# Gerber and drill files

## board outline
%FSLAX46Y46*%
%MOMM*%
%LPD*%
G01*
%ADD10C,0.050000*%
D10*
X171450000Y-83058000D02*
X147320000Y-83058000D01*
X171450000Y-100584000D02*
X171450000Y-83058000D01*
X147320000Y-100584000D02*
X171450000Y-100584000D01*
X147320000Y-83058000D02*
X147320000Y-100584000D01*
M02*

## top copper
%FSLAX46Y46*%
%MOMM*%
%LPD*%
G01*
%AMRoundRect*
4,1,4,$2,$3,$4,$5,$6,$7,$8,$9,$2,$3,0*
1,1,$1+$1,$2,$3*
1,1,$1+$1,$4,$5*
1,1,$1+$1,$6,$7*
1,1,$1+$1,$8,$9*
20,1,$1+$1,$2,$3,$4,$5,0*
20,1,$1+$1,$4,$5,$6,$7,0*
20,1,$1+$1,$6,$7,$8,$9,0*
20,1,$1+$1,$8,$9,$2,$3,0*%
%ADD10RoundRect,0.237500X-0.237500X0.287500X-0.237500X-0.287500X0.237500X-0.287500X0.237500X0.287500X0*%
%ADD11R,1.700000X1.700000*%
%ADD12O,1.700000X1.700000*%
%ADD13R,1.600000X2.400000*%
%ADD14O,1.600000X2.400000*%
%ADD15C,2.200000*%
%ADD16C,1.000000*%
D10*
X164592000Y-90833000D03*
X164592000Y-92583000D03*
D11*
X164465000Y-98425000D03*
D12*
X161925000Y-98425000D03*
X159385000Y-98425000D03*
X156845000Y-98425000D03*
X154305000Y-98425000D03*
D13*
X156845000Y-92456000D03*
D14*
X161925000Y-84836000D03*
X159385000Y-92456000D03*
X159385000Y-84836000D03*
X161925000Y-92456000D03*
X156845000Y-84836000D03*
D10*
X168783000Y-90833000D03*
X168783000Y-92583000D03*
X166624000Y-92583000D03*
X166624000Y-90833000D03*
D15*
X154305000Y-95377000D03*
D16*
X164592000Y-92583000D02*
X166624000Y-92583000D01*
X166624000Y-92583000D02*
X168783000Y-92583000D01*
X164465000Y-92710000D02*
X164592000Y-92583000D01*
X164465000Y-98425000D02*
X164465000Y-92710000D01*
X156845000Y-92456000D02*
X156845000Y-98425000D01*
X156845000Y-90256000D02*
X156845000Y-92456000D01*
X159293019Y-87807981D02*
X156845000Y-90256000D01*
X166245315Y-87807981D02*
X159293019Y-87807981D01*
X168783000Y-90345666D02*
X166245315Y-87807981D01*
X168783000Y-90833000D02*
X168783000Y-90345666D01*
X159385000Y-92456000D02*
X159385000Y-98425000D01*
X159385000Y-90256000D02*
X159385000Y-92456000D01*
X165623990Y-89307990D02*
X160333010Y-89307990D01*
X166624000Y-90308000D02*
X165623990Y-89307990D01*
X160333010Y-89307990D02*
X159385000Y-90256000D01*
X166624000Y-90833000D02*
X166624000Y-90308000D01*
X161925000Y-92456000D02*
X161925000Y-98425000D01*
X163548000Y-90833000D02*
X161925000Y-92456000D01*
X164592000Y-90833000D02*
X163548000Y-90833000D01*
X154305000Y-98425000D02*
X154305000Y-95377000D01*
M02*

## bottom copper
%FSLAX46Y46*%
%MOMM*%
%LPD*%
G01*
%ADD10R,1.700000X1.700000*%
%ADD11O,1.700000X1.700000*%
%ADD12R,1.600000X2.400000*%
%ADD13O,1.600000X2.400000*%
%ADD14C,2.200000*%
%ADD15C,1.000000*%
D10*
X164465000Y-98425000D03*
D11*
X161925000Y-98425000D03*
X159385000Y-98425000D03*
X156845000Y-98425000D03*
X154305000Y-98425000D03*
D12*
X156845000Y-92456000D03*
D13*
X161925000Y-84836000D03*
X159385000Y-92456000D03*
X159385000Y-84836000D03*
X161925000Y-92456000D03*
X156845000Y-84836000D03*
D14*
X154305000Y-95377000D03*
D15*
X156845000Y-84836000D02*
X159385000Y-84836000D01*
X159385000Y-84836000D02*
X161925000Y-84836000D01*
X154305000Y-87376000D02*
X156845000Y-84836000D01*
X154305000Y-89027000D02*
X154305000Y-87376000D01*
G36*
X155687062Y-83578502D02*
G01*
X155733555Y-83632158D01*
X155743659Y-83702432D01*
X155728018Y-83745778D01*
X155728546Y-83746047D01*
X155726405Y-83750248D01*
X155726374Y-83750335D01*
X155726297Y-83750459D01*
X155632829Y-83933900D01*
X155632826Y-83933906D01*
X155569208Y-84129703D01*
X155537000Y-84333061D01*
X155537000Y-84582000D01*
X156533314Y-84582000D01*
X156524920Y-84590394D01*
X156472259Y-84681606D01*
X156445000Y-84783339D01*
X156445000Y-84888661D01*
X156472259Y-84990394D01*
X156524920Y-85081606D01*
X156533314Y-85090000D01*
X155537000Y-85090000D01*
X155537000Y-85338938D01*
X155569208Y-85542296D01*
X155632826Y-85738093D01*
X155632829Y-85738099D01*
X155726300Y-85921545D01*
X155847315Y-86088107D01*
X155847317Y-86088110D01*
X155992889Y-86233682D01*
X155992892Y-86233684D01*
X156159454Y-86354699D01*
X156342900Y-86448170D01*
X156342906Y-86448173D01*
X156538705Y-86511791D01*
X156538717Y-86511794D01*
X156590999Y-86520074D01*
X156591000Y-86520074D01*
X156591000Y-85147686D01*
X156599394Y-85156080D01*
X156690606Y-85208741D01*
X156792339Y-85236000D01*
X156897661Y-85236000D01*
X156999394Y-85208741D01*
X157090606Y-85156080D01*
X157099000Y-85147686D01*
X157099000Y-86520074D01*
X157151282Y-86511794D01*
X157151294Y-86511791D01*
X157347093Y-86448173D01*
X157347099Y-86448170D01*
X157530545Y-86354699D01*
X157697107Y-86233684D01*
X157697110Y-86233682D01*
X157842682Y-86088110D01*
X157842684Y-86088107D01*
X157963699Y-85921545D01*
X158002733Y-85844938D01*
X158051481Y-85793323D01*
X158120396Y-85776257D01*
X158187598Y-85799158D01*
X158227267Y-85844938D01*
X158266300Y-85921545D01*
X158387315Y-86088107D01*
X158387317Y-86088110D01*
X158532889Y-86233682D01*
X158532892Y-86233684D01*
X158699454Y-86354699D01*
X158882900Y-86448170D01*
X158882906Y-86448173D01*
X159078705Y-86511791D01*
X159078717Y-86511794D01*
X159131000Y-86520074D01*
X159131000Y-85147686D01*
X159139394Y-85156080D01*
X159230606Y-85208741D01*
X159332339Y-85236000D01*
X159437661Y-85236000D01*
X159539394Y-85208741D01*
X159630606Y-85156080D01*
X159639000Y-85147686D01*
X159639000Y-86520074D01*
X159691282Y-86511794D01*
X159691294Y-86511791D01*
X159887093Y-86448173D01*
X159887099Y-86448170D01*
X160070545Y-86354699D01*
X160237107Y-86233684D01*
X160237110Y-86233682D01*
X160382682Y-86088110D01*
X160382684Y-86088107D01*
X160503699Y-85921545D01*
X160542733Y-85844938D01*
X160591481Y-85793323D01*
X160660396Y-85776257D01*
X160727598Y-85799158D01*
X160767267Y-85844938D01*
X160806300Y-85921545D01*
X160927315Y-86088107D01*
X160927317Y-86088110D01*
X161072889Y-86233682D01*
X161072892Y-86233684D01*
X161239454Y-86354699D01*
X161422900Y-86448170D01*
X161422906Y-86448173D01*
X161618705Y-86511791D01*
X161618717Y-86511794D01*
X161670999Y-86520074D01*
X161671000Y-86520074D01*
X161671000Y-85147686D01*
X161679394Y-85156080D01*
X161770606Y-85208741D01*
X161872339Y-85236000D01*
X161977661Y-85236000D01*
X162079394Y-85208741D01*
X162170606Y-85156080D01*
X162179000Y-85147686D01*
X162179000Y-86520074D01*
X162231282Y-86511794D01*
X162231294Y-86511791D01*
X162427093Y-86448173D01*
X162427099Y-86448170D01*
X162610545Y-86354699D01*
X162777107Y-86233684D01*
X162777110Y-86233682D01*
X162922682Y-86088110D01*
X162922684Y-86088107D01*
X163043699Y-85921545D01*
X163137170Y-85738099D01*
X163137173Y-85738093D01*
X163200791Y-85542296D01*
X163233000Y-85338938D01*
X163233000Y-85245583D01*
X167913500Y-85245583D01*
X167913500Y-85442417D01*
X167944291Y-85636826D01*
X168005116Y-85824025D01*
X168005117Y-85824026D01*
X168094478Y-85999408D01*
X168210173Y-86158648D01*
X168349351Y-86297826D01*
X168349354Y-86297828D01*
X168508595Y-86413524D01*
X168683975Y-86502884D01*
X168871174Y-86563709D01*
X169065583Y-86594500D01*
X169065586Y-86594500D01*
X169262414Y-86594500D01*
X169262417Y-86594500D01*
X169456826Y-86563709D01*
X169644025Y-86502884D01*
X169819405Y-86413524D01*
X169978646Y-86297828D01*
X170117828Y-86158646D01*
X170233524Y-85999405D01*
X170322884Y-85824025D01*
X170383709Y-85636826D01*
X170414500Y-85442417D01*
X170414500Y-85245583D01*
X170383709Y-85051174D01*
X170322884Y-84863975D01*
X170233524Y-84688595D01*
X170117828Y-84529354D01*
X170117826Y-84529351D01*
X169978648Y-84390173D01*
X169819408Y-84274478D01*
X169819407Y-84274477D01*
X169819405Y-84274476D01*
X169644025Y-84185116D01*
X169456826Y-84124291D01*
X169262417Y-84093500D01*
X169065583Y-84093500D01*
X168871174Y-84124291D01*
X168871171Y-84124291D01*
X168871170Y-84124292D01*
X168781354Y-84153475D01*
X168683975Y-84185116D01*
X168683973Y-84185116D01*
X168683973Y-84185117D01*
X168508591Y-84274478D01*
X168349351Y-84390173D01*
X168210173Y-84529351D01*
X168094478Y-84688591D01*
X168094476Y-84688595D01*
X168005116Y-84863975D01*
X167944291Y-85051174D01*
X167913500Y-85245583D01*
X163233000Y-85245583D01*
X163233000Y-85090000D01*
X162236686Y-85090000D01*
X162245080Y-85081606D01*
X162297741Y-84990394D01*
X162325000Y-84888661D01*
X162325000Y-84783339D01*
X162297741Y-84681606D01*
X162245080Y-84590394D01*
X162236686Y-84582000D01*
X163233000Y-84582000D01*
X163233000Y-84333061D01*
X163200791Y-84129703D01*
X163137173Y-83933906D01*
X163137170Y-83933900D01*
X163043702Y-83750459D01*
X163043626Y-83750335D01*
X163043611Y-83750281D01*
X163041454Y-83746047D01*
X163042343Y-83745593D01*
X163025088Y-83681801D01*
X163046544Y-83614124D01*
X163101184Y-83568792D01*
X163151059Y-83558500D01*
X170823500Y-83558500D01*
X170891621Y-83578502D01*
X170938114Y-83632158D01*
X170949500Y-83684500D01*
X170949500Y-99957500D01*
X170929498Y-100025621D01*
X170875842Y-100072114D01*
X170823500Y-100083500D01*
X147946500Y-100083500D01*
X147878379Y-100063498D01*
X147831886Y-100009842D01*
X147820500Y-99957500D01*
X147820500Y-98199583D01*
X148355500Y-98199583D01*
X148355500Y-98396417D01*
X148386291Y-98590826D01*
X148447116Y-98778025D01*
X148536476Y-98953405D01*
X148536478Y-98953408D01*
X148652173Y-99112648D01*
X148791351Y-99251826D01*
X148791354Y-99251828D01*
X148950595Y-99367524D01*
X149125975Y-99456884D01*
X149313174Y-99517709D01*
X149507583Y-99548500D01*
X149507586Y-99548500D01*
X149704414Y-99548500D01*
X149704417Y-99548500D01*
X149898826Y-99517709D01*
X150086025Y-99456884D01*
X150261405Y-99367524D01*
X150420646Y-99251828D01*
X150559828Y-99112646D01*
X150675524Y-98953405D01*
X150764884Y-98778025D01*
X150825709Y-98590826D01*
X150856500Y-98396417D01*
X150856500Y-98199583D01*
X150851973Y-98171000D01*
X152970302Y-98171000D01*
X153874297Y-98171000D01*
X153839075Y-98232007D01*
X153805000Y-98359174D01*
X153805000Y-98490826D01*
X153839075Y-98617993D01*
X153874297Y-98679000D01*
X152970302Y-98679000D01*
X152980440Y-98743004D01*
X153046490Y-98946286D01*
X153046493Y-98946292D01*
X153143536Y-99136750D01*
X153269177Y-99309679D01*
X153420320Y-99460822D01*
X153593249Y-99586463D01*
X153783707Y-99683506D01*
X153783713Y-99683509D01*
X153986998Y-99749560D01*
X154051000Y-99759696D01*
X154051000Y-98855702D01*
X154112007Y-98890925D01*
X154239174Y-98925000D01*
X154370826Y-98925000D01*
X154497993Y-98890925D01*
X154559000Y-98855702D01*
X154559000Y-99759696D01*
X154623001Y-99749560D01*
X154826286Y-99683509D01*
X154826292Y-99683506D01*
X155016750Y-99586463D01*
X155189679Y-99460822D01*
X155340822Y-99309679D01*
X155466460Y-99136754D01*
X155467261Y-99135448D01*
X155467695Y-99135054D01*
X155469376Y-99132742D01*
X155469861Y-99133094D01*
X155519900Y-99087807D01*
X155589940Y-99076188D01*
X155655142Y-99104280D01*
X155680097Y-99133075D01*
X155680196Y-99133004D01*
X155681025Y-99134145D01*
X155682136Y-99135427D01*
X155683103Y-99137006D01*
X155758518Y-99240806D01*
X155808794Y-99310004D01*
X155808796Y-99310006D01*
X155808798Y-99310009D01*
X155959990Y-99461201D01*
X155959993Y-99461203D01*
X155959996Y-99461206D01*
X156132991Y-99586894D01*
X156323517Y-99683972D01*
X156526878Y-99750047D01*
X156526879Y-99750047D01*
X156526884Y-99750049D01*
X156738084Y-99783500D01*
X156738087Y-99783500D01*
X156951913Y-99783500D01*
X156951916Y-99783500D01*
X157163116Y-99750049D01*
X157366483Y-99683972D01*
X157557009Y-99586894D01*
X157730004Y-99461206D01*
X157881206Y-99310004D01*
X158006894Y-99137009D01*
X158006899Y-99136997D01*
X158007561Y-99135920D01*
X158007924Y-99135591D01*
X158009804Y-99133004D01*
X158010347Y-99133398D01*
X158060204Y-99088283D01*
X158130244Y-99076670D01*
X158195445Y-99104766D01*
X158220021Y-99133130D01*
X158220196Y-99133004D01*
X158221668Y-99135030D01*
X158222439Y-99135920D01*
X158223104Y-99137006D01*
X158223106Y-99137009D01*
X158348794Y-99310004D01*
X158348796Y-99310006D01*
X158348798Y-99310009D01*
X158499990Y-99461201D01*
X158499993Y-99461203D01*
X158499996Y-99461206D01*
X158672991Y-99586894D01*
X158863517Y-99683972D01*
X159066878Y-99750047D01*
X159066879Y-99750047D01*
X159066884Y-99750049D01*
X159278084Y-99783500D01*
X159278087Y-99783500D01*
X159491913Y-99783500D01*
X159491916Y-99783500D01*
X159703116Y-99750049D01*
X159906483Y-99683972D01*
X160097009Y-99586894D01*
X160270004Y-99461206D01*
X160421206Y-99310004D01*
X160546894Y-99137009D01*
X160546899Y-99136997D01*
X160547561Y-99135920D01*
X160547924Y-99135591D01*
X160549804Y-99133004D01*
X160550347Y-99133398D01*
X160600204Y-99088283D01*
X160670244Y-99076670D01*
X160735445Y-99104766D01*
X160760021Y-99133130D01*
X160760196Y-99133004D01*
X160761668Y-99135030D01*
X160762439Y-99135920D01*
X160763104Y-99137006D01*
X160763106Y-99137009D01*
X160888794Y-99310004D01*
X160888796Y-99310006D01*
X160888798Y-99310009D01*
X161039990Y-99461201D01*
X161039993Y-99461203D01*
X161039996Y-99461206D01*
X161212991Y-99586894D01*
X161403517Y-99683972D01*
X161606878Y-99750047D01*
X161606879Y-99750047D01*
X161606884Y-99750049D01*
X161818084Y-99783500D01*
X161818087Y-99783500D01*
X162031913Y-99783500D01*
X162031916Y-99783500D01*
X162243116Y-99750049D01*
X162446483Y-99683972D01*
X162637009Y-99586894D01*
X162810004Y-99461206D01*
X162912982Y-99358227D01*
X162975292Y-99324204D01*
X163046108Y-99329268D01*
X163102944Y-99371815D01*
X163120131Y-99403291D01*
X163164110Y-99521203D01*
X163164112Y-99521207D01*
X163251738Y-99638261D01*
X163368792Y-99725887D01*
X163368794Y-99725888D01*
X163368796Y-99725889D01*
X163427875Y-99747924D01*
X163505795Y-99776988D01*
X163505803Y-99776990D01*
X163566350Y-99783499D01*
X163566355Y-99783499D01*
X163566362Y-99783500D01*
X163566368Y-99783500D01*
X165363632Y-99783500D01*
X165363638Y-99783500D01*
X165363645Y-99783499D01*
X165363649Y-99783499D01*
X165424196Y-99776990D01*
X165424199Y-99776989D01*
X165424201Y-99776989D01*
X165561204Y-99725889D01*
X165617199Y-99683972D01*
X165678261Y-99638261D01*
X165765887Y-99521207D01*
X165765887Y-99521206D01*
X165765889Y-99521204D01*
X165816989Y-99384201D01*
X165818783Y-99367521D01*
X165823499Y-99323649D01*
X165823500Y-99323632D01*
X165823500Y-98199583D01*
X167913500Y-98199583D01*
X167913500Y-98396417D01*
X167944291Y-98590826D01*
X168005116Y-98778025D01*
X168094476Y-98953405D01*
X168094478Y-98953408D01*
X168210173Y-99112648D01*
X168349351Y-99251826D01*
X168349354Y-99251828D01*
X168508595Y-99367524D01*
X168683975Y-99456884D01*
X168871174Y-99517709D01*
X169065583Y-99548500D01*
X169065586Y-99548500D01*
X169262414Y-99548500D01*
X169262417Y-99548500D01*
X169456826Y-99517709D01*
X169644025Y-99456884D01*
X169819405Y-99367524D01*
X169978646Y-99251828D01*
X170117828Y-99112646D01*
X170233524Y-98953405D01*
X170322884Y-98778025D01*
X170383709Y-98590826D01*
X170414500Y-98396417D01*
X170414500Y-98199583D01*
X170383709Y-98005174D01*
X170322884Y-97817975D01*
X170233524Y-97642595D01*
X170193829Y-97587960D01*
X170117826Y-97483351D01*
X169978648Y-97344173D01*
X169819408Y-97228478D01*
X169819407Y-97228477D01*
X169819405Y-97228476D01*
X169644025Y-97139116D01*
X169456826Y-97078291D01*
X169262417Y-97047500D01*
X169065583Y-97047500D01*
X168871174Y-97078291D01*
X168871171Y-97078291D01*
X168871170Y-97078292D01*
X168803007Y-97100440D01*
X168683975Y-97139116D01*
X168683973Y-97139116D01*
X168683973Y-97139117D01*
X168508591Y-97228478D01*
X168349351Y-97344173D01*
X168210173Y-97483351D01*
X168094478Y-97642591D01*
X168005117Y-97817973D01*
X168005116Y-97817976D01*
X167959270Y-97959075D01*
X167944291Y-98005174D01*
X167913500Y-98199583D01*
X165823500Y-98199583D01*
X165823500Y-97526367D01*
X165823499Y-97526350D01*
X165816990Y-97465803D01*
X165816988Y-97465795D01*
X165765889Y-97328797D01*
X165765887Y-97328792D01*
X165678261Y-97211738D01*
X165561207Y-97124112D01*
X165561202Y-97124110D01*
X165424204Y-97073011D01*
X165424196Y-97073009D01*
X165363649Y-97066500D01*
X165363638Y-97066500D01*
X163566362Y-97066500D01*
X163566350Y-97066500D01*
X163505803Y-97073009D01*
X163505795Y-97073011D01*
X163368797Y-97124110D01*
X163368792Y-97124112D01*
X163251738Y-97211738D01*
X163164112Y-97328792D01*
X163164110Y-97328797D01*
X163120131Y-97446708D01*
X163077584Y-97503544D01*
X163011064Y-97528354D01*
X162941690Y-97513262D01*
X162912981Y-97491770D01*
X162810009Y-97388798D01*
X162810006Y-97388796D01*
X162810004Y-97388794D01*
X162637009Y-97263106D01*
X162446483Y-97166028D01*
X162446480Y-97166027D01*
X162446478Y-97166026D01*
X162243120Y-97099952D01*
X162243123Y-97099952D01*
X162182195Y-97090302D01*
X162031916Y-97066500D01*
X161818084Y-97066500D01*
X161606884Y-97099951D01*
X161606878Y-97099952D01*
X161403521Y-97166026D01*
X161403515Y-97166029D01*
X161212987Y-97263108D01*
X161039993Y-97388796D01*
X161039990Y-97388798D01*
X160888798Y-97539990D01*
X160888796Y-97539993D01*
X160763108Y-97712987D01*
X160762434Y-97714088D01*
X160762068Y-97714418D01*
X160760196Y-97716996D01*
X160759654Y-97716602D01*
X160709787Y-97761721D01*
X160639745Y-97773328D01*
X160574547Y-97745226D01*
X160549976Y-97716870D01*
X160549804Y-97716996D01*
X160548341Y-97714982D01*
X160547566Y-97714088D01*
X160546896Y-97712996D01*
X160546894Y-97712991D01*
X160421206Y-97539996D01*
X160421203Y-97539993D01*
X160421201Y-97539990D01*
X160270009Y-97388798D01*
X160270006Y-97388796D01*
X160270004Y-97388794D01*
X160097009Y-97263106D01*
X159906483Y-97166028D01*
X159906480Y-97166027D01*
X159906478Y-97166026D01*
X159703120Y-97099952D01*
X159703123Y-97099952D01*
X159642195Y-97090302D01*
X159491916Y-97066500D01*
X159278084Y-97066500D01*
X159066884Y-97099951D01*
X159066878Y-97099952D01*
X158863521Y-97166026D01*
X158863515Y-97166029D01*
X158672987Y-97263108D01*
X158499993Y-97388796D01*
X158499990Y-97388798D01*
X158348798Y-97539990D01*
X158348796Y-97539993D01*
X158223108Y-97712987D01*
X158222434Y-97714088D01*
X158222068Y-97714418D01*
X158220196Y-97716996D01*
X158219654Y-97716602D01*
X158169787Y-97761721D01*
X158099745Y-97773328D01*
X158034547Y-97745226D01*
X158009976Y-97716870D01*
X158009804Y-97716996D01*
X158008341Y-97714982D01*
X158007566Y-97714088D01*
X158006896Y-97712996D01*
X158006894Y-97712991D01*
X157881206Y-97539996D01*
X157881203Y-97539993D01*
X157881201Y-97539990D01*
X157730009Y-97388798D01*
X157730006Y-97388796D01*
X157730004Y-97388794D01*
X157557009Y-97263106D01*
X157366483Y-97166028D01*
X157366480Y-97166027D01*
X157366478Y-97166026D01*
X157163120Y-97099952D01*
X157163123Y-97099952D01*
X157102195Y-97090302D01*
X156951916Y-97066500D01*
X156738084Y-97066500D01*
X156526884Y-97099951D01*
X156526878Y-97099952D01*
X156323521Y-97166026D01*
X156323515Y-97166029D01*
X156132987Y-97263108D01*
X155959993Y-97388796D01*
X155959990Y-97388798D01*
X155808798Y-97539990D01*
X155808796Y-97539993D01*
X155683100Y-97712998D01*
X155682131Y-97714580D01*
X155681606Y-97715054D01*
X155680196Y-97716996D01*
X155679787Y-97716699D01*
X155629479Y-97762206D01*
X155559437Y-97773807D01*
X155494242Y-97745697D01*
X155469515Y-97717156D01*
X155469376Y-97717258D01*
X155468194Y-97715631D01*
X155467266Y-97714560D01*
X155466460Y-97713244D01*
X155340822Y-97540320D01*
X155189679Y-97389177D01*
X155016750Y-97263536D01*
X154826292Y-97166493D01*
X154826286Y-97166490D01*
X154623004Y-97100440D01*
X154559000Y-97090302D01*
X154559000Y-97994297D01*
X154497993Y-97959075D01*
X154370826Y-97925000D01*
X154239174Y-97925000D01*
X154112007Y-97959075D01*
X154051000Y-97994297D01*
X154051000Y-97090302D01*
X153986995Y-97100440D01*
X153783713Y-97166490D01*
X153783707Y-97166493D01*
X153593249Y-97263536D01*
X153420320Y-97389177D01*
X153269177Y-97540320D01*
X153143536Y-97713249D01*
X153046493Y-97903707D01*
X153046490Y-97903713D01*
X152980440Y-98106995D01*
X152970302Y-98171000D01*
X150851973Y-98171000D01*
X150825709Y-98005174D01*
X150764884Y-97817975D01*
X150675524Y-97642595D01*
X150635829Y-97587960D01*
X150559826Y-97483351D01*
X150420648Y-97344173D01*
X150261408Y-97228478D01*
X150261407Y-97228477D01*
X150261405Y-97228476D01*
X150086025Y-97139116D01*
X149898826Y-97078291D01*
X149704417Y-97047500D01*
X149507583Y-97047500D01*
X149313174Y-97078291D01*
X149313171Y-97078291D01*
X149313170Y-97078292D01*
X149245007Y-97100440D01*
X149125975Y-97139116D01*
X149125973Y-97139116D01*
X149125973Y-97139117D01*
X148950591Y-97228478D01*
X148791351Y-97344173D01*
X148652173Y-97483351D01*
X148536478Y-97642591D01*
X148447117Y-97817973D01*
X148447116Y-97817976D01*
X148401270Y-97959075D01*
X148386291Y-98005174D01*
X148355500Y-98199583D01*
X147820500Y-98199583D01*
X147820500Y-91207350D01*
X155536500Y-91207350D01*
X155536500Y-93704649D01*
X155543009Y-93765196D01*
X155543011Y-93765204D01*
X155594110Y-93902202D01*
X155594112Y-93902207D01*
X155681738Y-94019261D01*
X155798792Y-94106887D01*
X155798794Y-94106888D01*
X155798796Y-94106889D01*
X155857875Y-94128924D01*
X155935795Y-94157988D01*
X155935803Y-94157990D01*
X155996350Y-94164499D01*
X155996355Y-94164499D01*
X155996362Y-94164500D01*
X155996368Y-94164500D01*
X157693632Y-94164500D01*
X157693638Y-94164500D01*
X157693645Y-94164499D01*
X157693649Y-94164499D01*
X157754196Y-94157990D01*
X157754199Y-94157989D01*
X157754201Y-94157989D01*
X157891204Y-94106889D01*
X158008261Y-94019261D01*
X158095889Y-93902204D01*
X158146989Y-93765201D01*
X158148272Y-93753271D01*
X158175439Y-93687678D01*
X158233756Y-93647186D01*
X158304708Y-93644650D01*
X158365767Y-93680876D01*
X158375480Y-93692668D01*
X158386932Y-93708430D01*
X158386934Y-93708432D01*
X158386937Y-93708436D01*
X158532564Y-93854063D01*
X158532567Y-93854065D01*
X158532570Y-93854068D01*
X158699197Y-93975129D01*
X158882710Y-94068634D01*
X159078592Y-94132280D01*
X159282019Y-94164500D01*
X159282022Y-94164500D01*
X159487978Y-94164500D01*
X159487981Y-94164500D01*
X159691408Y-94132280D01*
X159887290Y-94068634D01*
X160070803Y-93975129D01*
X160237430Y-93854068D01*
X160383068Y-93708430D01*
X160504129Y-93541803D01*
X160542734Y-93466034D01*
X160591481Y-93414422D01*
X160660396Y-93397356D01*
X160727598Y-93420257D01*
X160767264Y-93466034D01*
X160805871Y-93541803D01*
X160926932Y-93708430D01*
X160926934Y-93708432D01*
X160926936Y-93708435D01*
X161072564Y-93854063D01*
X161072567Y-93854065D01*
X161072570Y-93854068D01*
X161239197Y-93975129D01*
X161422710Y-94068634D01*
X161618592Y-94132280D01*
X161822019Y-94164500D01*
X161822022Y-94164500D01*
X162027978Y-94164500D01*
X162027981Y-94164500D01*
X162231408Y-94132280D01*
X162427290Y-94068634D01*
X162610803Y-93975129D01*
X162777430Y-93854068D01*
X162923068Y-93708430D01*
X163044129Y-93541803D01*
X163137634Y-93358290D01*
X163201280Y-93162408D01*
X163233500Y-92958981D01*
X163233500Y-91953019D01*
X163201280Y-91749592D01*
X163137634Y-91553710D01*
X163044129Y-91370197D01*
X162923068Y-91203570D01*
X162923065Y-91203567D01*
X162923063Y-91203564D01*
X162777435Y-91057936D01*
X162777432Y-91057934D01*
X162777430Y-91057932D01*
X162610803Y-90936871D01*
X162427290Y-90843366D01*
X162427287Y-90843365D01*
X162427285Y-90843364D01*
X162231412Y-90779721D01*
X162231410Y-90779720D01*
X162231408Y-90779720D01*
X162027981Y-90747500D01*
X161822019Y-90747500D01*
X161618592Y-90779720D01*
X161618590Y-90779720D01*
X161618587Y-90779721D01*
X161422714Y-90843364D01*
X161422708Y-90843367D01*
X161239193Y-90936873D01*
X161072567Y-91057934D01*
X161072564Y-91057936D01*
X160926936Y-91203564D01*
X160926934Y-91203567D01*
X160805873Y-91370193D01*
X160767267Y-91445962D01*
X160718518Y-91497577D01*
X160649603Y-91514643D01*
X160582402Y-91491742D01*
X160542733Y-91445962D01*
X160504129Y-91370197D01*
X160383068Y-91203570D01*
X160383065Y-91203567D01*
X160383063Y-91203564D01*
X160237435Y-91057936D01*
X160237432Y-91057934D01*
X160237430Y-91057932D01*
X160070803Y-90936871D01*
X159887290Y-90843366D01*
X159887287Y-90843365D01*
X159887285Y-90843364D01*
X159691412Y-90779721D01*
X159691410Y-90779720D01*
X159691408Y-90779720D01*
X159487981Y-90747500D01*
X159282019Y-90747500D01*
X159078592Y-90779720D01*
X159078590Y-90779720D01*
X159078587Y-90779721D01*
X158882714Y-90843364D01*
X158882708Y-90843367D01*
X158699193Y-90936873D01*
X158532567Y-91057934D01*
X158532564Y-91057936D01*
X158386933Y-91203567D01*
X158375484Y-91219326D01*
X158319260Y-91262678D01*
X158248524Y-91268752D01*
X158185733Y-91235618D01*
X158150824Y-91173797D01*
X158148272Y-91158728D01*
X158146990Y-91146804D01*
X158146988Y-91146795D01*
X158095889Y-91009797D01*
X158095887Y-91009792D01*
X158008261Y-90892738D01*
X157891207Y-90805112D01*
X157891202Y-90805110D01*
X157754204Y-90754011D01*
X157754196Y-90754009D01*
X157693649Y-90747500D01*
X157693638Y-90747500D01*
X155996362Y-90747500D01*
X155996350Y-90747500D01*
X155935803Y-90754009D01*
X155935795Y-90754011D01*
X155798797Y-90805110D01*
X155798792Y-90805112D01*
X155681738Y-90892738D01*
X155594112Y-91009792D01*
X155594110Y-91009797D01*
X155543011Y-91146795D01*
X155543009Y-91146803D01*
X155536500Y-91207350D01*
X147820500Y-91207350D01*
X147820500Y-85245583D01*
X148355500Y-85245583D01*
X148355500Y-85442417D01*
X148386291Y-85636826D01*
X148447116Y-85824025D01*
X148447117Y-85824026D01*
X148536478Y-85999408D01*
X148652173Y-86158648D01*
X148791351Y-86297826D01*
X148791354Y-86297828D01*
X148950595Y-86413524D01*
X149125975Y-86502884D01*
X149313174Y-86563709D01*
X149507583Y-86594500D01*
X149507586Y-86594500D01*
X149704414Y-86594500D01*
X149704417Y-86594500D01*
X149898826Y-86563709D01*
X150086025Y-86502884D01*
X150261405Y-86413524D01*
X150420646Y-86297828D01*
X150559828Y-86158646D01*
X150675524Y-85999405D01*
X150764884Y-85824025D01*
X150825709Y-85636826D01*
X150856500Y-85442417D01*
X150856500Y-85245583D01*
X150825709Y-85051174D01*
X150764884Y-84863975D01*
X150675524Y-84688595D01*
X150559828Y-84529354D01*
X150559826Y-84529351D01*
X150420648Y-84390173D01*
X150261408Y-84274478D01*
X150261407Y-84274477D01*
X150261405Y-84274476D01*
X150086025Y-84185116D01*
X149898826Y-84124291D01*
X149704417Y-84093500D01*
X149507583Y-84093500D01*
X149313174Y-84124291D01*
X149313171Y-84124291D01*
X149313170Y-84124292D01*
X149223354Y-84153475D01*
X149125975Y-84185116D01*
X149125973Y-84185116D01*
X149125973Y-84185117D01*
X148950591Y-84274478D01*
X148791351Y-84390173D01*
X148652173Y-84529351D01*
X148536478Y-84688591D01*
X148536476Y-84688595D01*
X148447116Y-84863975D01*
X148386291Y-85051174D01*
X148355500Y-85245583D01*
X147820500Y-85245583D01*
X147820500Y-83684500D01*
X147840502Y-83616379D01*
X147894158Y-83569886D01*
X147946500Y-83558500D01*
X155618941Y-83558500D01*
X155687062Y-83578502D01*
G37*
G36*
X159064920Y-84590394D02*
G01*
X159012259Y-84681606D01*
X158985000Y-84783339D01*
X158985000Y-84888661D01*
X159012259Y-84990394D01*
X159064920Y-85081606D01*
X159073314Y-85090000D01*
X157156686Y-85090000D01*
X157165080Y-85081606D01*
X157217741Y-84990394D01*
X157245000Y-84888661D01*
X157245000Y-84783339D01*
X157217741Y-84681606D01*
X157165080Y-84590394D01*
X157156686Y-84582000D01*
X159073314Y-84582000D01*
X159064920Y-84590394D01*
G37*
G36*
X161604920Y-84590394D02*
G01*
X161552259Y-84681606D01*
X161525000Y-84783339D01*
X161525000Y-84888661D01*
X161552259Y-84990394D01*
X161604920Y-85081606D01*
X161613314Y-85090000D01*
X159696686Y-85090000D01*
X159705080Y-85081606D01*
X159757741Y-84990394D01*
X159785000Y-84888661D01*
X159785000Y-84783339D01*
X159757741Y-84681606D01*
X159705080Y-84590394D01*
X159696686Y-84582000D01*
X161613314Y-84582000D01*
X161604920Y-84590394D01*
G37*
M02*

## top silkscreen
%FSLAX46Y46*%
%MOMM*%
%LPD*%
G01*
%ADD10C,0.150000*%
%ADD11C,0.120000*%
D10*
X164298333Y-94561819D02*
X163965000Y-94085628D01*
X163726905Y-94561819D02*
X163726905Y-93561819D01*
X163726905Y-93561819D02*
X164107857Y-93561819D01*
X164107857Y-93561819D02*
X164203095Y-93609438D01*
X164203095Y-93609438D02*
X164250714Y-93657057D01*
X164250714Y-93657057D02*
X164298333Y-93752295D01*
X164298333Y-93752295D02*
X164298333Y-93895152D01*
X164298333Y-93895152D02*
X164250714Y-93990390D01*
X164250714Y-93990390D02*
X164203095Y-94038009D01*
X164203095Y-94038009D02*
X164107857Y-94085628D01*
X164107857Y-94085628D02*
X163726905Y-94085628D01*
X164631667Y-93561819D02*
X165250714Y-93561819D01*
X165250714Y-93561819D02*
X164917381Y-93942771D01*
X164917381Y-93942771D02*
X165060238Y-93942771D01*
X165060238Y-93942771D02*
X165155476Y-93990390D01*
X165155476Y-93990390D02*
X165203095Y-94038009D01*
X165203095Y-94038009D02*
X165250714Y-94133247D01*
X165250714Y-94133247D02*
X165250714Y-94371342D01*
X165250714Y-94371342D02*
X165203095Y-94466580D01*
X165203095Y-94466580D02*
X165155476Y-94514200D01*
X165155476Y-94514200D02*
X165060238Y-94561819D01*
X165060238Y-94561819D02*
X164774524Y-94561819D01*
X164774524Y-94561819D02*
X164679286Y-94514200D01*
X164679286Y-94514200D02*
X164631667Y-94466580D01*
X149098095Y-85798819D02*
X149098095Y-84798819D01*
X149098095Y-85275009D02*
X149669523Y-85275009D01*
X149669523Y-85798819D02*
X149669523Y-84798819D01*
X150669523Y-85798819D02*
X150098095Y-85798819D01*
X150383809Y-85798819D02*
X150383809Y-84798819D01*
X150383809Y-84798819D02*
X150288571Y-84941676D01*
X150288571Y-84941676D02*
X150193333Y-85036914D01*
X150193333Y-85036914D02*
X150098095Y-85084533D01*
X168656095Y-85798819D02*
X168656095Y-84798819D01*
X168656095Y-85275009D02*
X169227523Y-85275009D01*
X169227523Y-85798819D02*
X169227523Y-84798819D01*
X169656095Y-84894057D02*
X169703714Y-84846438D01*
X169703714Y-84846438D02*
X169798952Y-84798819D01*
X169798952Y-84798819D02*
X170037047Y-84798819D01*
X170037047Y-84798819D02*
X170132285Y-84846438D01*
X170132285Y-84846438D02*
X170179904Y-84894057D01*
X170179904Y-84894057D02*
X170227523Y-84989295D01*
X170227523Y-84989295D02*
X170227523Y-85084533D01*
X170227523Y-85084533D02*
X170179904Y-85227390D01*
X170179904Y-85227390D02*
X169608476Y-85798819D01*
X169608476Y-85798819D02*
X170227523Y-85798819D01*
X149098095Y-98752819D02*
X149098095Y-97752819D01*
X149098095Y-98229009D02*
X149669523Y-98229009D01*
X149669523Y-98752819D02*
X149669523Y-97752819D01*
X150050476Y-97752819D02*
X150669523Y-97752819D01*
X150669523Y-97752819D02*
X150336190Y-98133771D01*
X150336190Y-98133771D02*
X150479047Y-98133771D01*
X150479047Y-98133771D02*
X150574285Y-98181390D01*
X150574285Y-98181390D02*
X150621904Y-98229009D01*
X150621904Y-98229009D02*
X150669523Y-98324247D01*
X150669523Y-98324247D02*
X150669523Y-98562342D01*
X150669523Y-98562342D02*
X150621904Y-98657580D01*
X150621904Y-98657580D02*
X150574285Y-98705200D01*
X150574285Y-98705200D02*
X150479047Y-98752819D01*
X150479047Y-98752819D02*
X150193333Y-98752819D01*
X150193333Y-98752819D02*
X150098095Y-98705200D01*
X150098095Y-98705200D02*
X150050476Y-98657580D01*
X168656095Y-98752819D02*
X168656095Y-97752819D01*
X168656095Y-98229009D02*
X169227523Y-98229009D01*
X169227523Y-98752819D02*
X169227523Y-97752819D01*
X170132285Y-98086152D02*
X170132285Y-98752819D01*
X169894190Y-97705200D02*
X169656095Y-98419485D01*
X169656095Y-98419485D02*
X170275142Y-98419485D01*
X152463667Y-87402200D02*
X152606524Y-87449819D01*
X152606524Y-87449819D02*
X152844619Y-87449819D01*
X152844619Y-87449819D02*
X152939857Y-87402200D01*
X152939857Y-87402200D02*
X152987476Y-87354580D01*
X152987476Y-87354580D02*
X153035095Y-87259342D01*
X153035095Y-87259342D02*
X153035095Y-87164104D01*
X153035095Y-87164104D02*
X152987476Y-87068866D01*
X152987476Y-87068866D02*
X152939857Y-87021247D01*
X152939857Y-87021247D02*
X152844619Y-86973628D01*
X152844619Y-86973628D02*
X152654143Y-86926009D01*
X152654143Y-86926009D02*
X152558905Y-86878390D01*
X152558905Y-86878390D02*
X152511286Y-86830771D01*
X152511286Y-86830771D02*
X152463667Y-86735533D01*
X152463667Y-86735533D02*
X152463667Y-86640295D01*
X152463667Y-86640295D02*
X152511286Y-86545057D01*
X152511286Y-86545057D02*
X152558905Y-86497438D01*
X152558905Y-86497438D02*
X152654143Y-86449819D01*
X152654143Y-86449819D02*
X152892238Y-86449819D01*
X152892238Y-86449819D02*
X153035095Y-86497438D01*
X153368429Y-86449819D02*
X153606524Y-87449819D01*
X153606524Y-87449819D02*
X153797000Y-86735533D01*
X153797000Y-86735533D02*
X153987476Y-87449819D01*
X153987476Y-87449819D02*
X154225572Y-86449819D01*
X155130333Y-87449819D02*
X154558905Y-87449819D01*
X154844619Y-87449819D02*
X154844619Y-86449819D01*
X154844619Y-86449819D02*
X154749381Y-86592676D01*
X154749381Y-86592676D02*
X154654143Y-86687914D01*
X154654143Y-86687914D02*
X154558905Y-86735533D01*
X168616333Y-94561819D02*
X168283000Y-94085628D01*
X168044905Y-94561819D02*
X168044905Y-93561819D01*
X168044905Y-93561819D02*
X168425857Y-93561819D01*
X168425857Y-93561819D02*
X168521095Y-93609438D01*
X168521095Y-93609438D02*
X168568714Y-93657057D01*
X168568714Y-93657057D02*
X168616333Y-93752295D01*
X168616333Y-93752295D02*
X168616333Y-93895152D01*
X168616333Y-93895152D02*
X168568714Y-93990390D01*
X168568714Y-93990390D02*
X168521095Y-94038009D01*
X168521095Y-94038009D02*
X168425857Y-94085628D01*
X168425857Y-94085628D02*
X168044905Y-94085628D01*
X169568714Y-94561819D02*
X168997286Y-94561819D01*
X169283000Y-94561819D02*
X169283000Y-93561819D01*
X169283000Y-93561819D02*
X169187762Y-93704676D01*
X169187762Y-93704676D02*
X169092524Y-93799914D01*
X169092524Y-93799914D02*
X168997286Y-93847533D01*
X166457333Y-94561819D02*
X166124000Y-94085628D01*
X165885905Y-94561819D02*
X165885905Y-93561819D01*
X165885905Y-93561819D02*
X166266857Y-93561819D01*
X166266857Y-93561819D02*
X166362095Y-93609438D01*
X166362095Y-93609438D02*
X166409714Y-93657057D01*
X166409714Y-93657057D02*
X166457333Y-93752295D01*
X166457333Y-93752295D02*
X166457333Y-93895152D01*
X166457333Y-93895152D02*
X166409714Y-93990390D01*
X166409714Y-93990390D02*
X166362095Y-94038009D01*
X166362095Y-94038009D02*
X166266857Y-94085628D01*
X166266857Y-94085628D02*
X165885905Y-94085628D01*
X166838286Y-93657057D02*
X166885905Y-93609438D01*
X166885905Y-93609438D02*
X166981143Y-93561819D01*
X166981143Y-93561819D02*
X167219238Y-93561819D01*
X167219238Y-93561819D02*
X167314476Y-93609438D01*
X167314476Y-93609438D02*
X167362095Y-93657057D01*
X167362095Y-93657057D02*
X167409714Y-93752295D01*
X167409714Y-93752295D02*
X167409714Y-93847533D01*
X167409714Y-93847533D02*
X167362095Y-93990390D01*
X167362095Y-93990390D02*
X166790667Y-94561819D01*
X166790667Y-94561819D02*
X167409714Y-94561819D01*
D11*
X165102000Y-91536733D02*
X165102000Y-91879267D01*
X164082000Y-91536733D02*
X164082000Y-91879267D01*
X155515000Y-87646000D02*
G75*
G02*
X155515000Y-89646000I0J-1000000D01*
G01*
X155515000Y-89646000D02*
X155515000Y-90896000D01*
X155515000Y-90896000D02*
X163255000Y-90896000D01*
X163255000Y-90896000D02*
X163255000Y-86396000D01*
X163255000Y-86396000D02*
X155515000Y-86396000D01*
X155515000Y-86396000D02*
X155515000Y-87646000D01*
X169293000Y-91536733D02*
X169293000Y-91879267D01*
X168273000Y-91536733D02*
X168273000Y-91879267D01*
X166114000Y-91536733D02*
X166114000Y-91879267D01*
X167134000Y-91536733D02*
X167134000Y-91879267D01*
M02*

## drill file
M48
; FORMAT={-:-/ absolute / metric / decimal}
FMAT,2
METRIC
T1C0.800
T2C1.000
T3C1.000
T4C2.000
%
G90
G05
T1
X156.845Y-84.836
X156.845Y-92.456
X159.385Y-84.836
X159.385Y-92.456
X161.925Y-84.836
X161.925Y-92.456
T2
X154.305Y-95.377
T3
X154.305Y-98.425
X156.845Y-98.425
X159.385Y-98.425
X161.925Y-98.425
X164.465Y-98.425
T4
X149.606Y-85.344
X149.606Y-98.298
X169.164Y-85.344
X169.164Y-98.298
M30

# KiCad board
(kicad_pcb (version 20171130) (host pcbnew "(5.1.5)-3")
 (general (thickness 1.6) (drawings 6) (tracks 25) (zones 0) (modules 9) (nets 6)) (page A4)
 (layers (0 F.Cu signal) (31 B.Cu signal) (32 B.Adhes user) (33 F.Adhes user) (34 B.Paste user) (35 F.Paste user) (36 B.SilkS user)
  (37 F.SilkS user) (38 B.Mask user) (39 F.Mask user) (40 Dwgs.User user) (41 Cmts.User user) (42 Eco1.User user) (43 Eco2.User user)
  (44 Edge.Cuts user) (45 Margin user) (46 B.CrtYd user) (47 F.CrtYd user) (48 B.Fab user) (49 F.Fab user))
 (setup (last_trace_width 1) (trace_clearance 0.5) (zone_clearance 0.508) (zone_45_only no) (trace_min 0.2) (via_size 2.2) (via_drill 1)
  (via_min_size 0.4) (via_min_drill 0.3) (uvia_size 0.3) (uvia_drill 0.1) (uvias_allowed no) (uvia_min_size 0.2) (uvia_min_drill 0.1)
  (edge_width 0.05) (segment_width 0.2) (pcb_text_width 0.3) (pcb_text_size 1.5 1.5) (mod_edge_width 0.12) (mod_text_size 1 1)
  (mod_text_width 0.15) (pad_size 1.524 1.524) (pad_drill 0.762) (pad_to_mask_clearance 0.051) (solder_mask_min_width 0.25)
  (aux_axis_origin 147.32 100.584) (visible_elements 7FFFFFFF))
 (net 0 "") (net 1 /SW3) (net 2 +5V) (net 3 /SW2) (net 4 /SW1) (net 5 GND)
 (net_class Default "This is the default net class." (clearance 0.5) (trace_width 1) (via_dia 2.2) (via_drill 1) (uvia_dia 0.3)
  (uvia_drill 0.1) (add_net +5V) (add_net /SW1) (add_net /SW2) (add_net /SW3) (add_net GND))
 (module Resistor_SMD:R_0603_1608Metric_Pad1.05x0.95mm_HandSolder (layer F.Cu) (at 164.592 91.708 270)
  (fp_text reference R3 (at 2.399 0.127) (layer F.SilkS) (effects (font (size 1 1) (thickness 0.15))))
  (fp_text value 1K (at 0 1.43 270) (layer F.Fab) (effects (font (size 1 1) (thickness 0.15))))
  (fp_line (start -0.171267 -0.51) (end 0.171267 -0.51) (layer F.SilkS) (width 0.12))
  (fp_line (start -0.171267 0.51) (end 0.171267 0.51) (layer F.SilkS) (width 0.12))
  (pad 1 smd roundrect (at -0.875 0 270) (size 1.05 0.95) (layers F.Cu F.Paste F.Mask) (roundrect_rratio 0.25) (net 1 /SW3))
  (pad 2 smd roundrect (at 0.875 0 270) (size 1.05 0.95) (layers F.Cu F.Paste F.Mask) (roundrect_rratio 0.25) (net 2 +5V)))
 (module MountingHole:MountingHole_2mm (layer F.Cu) (at 149.606 85.344)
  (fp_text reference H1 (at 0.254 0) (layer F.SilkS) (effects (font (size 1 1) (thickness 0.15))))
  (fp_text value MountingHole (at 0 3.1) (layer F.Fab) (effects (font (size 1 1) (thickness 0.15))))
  (pad "" np_thru_hole circle (at 0 0) (size 2 2) (drill 2) (layers *.Cu *.Mask)))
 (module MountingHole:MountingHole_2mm (layer F.Cu) (at 169.164 85.344)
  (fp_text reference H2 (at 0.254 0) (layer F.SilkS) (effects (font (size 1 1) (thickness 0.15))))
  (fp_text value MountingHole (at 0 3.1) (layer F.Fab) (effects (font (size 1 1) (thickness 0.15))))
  (pad "" np_thru_hole circle (at 0 0) (size 2 2) (drill 2) (layers *.Cu *.Mask)))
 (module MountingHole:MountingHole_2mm (layer F.Cu) (at 149.606 98.298)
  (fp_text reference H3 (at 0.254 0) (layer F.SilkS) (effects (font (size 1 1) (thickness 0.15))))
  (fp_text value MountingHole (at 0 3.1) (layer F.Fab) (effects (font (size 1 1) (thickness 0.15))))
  (pad "" np_thru_hole circle (at 0 0) (size 2 2) (drill 2) (layers *.Cu *.Mask)))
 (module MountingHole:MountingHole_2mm (layer F.Cu) (at 169.164 98.298)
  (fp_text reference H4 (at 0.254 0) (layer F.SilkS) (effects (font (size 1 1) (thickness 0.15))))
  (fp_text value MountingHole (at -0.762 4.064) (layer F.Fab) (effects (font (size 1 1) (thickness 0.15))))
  (pad "" np_thru_hole circle (at 0 0) (size 2 2) (drill 2) (layers *.Cu *.Mask)))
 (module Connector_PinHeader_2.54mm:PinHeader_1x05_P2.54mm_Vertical (layer B.Cu) (at 164.465 98.425 90)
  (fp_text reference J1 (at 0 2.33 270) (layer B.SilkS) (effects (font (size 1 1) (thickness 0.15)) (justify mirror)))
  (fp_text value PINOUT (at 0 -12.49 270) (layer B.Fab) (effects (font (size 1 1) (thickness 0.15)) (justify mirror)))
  (pad 1 thru_hole rect (at 0 0 90) (size 1.7 1.7) (drill 1) (layers *.Cu *.Mask) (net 2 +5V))
  (pad 2 thru_hole oval (at 0 -2.54 90) (size 1.7 1.7) (drill 1) (layers *.Cu *.Mask) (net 1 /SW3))
  (pad 3 thru_hole oval (at 0 -5.08 90) (size 1.7 1.7) (drill 1) (layers *.Cu *.Mask) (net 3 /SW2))
  (pad 4 thru_hole oval (at 0 -7.62 90) (size 1.7 1.7) (drill 1) (layers *.Cu *.Mask) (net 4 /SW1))
  (pad 5 thru_hole oval (at 0 -10.16 90) (size 1.7 1.7) (drill 1) (layers *.Cu *.Mask) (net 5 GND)))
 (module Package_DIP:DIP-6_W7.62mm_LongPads (layer F.Cu) (at 156.845 92.456 90)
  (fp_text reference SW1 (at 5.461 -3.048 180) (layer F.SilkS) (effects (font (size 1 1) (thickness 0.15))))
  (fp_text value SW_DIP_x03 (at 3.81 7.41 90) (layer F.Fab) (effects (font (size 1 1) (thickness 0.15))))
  (fp_arc (start 3.81 -1.33) (end 2.81 -1.33) (angle -180) (layer F.SilkS) (width 0.12))
  (fp_line (start 2.81 -1.33) (end 1.56 -1.33) (layer F.SilkS) (width 0.12))
  (fp_line (start 1.56 -1.33) (end 1.56 6.41) (layer F.SilkS) (width 0.12))
  (fp_line (start 1.56 6.41) (end 6.06 6.41) (layer F.SilkS) (width 0.12))
  (fp_line (start 6.06 6.41) (end 6.06 -1.33) (layer F.SilkS) (width 0.12))
  (fp_line (start 6.06 -1.33) (end 4.81 -1.33) (layer F.SilkS) (width 0.12))
  (pad 1 thru_hole rect (at 0 0 90) (size 2.4 1.6) (drill 0.8) (layers *.Cu *.Mask) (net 4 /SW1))
  (pad 4 thru_hole oval (at 7.62 5.08 90) (size 2.4 1.6) (drill 0.8) (layers *.Cu *.Mask) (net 5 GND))
  (pad 2 thru_hole oval (at 0 2.54 90) (size 2.4 1.6) (drill 0.8) (layers *.Cu *.Mask) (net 3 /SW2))
  (pad 5 thru_hole oval (at 7.62 2.54 90) (size 2.4 1.6) (drill 0.8) (layers *.Cu *.Mask) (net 5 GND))
  (pad 3 thru_hole oval (at 0 5.08 90) (size 2.4 1.6) (drill 0.8) (layers *.Cu *.Mask) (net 1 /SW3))
  (pad 6 thru_hole oval (at 7.62 0 90) (size 2.4 1.6) (drill 0.8) (layers *.Cu *.Mask) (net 5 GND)))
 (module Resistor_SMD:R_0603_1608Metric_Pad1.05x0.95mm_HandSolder (layer F.Cu) (at 168.783 91.708 270)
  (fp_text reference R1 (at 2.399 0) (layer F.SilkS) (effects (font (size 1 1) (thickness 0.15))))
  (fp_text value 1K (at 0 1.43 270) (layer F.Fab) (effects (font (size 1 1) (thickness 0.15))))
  (fp_line (start -0.171267 -0.51) (end 0.171267 -0.51) (layer F.SilkS) (width 0.12))
  (fp_line (start -0.171267 0.51) (end 0.171267 0.51) (layer F.SilkS) (width 0.12))
  (pad 1 smd roundrect (at -0.875 0 270) (size 1.05 0.95) (layers F.Cu F.Paste F.Mask) (roundrect_rratio 0.25) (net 4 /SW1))
  (pad 2 smd roundrect (at 0.875 0 270) (size 1.05 0.95) (layers F.Cu F.Paste F.Mask) (roundrect_rratio 0.25) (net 2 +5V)))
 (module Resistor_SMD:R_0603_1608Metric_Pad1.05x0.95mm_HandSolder (layer F.Cu) (at 166.624 91.708 270)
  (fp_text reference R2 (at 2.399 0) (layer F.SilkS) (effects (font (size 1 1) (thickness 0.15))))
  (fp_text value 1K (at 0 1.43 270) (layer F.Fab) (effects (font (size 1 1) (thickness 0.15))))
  (fp_line (start -0.171267 0.51) (end 0.171267 0.51) (layer F.SilkS) (width 0.12))
  (fp_line (start -0.171267 -0.51) (end 0.171267 -0.51) (layer F.SilkS) (width 0.12))
  (pad 2 smd roundrect (at 0.875 0 270) (size 1.05 0.95) (layers F.Cu F.Paste F.Mask) (roundrect_rratio 0.25) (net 2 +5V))
  (pad 1 smd roundrect (at -0.875 0 270) (size 1.05 0.95) (layers F.Cu F.Paste F.Mask) (roundrect_rratio 0.25) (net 3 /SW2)))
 (gr_line (start 171.45 83.058) (end 147.32 83.058) (layer Edge.Cuts) (width 0.05))
 (gr_line (start 171.45 100.584) (end 171.45 83.058) (layer Edge.Cuts) (width 0.05))
 (gr_line (start 147.32 100.584) (end 171.45 100.584) (layer Edge.Cuts) (width 0.05))
 (gr_line (start 147.32 83.058) (end 147.32 100.584) (layer Edge.Cuts) (width 0.05))
 (segment (start 164.592 92.583) (end 166.624 92.583) (width 1) (layer F.Cu) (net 2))
 (segment (start 166.624 92.583) (end 168.783 92.583) (width 1) (layer F.Cu) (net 2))
 (segment (start 164.465 92.71) (end 164.592 92.583) (width 1) (layer F.Cu) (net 2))
 (segment (start 164.465 98.425) (end 164.465 92.71) (width 1) (layer F.Cu) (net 2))
 (segment (start 156.845 92.456) (end 156.845 98.425) (width 1) (layer F.Cu) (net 4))
 (segment (start 156.845 90.256) (end 156.845 92.456) (width 1) (layer F.Cu) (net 4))
 (segment (start 159.293019 87.807981) (end 156.845 90.256) (width 1) (layer F.Cu) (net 4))
 (segment (start 166.245315 87.807981) (end 159.293019 87.807981) (width 1) (layer F.Cu) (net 4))
 (segment (start 168.783 90.345666) (end 166.245315 87.807981) (width 1) (layer F.Cu) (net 4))
 (segment (start 168.783 90.833) (end 168.783 90.345666) (width 1) (layer F.Cu) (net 4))
 (segment (start 159.385 92.456) (end 159.385 98.425) (width 1) (layer F.Cu) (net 3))
 (segment (start 159.385 90.256) (end 159.385 92.456) (width 1) (layer F.Cu) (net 3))
 (segment (start 165.62399 89.30799) (end 160.33301 89.30799) (width 1) (layer F.Cu) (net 3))
 (segment (start 166.624 90.308) (end 165.62399 89.30799) (width 1) (layer F.Cu) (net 3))
 (segment (start 160.33301 89.30799) (end 159.385 90.256) (width 1) (layer F.Cu) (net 3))
 (segment (start 166.624 90.833) (end 166.624 90.308) (width 1) (layer F.Cu) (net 3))
 (segment (start 161.925 92.456) (end 161.925 98.425) (width 1) (layer F.Cu) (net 1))
 (segment (start 163.548 90.833) (end 161.925 92.456) (width 1) (layer F.Cu) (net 1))
 (segment (start 164.592 90.833) (end 163.548 90.833) (width 1) (layer F.Cu) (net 1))
 (segment (start 156.845 84.836) (end 159.385 84.836) (width 1) (layer B.Cu) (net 5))
 (segment (start 159.385 84.836) (end 161.925 84.836) (width 1) (layer B.Cu) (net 5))
 (segment (start 154.305 87.376) (end 156.845 84.836) (width 1) (layer B.Cu) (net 5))
 (segment (start 154.305 89.027) (end 154.305 87.376) (width 1) (layer B.Cu) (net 5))
 (via (at 154.305 95.377) (size 2.2) (drill 1) (layers F.Cu B.Cu) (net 5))
 (segment (start 154.305 98.425) (end 154.305 95.377) (width 1) (layer F.Cu) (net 5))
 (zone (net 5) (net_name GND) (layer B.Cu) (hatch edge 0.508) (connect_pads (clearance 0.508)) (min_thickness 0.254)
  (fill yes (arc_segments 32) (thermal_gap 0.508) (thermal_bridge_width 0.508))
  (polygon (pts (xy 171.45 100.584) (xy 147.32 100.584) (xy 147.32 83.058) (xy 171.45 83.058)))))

